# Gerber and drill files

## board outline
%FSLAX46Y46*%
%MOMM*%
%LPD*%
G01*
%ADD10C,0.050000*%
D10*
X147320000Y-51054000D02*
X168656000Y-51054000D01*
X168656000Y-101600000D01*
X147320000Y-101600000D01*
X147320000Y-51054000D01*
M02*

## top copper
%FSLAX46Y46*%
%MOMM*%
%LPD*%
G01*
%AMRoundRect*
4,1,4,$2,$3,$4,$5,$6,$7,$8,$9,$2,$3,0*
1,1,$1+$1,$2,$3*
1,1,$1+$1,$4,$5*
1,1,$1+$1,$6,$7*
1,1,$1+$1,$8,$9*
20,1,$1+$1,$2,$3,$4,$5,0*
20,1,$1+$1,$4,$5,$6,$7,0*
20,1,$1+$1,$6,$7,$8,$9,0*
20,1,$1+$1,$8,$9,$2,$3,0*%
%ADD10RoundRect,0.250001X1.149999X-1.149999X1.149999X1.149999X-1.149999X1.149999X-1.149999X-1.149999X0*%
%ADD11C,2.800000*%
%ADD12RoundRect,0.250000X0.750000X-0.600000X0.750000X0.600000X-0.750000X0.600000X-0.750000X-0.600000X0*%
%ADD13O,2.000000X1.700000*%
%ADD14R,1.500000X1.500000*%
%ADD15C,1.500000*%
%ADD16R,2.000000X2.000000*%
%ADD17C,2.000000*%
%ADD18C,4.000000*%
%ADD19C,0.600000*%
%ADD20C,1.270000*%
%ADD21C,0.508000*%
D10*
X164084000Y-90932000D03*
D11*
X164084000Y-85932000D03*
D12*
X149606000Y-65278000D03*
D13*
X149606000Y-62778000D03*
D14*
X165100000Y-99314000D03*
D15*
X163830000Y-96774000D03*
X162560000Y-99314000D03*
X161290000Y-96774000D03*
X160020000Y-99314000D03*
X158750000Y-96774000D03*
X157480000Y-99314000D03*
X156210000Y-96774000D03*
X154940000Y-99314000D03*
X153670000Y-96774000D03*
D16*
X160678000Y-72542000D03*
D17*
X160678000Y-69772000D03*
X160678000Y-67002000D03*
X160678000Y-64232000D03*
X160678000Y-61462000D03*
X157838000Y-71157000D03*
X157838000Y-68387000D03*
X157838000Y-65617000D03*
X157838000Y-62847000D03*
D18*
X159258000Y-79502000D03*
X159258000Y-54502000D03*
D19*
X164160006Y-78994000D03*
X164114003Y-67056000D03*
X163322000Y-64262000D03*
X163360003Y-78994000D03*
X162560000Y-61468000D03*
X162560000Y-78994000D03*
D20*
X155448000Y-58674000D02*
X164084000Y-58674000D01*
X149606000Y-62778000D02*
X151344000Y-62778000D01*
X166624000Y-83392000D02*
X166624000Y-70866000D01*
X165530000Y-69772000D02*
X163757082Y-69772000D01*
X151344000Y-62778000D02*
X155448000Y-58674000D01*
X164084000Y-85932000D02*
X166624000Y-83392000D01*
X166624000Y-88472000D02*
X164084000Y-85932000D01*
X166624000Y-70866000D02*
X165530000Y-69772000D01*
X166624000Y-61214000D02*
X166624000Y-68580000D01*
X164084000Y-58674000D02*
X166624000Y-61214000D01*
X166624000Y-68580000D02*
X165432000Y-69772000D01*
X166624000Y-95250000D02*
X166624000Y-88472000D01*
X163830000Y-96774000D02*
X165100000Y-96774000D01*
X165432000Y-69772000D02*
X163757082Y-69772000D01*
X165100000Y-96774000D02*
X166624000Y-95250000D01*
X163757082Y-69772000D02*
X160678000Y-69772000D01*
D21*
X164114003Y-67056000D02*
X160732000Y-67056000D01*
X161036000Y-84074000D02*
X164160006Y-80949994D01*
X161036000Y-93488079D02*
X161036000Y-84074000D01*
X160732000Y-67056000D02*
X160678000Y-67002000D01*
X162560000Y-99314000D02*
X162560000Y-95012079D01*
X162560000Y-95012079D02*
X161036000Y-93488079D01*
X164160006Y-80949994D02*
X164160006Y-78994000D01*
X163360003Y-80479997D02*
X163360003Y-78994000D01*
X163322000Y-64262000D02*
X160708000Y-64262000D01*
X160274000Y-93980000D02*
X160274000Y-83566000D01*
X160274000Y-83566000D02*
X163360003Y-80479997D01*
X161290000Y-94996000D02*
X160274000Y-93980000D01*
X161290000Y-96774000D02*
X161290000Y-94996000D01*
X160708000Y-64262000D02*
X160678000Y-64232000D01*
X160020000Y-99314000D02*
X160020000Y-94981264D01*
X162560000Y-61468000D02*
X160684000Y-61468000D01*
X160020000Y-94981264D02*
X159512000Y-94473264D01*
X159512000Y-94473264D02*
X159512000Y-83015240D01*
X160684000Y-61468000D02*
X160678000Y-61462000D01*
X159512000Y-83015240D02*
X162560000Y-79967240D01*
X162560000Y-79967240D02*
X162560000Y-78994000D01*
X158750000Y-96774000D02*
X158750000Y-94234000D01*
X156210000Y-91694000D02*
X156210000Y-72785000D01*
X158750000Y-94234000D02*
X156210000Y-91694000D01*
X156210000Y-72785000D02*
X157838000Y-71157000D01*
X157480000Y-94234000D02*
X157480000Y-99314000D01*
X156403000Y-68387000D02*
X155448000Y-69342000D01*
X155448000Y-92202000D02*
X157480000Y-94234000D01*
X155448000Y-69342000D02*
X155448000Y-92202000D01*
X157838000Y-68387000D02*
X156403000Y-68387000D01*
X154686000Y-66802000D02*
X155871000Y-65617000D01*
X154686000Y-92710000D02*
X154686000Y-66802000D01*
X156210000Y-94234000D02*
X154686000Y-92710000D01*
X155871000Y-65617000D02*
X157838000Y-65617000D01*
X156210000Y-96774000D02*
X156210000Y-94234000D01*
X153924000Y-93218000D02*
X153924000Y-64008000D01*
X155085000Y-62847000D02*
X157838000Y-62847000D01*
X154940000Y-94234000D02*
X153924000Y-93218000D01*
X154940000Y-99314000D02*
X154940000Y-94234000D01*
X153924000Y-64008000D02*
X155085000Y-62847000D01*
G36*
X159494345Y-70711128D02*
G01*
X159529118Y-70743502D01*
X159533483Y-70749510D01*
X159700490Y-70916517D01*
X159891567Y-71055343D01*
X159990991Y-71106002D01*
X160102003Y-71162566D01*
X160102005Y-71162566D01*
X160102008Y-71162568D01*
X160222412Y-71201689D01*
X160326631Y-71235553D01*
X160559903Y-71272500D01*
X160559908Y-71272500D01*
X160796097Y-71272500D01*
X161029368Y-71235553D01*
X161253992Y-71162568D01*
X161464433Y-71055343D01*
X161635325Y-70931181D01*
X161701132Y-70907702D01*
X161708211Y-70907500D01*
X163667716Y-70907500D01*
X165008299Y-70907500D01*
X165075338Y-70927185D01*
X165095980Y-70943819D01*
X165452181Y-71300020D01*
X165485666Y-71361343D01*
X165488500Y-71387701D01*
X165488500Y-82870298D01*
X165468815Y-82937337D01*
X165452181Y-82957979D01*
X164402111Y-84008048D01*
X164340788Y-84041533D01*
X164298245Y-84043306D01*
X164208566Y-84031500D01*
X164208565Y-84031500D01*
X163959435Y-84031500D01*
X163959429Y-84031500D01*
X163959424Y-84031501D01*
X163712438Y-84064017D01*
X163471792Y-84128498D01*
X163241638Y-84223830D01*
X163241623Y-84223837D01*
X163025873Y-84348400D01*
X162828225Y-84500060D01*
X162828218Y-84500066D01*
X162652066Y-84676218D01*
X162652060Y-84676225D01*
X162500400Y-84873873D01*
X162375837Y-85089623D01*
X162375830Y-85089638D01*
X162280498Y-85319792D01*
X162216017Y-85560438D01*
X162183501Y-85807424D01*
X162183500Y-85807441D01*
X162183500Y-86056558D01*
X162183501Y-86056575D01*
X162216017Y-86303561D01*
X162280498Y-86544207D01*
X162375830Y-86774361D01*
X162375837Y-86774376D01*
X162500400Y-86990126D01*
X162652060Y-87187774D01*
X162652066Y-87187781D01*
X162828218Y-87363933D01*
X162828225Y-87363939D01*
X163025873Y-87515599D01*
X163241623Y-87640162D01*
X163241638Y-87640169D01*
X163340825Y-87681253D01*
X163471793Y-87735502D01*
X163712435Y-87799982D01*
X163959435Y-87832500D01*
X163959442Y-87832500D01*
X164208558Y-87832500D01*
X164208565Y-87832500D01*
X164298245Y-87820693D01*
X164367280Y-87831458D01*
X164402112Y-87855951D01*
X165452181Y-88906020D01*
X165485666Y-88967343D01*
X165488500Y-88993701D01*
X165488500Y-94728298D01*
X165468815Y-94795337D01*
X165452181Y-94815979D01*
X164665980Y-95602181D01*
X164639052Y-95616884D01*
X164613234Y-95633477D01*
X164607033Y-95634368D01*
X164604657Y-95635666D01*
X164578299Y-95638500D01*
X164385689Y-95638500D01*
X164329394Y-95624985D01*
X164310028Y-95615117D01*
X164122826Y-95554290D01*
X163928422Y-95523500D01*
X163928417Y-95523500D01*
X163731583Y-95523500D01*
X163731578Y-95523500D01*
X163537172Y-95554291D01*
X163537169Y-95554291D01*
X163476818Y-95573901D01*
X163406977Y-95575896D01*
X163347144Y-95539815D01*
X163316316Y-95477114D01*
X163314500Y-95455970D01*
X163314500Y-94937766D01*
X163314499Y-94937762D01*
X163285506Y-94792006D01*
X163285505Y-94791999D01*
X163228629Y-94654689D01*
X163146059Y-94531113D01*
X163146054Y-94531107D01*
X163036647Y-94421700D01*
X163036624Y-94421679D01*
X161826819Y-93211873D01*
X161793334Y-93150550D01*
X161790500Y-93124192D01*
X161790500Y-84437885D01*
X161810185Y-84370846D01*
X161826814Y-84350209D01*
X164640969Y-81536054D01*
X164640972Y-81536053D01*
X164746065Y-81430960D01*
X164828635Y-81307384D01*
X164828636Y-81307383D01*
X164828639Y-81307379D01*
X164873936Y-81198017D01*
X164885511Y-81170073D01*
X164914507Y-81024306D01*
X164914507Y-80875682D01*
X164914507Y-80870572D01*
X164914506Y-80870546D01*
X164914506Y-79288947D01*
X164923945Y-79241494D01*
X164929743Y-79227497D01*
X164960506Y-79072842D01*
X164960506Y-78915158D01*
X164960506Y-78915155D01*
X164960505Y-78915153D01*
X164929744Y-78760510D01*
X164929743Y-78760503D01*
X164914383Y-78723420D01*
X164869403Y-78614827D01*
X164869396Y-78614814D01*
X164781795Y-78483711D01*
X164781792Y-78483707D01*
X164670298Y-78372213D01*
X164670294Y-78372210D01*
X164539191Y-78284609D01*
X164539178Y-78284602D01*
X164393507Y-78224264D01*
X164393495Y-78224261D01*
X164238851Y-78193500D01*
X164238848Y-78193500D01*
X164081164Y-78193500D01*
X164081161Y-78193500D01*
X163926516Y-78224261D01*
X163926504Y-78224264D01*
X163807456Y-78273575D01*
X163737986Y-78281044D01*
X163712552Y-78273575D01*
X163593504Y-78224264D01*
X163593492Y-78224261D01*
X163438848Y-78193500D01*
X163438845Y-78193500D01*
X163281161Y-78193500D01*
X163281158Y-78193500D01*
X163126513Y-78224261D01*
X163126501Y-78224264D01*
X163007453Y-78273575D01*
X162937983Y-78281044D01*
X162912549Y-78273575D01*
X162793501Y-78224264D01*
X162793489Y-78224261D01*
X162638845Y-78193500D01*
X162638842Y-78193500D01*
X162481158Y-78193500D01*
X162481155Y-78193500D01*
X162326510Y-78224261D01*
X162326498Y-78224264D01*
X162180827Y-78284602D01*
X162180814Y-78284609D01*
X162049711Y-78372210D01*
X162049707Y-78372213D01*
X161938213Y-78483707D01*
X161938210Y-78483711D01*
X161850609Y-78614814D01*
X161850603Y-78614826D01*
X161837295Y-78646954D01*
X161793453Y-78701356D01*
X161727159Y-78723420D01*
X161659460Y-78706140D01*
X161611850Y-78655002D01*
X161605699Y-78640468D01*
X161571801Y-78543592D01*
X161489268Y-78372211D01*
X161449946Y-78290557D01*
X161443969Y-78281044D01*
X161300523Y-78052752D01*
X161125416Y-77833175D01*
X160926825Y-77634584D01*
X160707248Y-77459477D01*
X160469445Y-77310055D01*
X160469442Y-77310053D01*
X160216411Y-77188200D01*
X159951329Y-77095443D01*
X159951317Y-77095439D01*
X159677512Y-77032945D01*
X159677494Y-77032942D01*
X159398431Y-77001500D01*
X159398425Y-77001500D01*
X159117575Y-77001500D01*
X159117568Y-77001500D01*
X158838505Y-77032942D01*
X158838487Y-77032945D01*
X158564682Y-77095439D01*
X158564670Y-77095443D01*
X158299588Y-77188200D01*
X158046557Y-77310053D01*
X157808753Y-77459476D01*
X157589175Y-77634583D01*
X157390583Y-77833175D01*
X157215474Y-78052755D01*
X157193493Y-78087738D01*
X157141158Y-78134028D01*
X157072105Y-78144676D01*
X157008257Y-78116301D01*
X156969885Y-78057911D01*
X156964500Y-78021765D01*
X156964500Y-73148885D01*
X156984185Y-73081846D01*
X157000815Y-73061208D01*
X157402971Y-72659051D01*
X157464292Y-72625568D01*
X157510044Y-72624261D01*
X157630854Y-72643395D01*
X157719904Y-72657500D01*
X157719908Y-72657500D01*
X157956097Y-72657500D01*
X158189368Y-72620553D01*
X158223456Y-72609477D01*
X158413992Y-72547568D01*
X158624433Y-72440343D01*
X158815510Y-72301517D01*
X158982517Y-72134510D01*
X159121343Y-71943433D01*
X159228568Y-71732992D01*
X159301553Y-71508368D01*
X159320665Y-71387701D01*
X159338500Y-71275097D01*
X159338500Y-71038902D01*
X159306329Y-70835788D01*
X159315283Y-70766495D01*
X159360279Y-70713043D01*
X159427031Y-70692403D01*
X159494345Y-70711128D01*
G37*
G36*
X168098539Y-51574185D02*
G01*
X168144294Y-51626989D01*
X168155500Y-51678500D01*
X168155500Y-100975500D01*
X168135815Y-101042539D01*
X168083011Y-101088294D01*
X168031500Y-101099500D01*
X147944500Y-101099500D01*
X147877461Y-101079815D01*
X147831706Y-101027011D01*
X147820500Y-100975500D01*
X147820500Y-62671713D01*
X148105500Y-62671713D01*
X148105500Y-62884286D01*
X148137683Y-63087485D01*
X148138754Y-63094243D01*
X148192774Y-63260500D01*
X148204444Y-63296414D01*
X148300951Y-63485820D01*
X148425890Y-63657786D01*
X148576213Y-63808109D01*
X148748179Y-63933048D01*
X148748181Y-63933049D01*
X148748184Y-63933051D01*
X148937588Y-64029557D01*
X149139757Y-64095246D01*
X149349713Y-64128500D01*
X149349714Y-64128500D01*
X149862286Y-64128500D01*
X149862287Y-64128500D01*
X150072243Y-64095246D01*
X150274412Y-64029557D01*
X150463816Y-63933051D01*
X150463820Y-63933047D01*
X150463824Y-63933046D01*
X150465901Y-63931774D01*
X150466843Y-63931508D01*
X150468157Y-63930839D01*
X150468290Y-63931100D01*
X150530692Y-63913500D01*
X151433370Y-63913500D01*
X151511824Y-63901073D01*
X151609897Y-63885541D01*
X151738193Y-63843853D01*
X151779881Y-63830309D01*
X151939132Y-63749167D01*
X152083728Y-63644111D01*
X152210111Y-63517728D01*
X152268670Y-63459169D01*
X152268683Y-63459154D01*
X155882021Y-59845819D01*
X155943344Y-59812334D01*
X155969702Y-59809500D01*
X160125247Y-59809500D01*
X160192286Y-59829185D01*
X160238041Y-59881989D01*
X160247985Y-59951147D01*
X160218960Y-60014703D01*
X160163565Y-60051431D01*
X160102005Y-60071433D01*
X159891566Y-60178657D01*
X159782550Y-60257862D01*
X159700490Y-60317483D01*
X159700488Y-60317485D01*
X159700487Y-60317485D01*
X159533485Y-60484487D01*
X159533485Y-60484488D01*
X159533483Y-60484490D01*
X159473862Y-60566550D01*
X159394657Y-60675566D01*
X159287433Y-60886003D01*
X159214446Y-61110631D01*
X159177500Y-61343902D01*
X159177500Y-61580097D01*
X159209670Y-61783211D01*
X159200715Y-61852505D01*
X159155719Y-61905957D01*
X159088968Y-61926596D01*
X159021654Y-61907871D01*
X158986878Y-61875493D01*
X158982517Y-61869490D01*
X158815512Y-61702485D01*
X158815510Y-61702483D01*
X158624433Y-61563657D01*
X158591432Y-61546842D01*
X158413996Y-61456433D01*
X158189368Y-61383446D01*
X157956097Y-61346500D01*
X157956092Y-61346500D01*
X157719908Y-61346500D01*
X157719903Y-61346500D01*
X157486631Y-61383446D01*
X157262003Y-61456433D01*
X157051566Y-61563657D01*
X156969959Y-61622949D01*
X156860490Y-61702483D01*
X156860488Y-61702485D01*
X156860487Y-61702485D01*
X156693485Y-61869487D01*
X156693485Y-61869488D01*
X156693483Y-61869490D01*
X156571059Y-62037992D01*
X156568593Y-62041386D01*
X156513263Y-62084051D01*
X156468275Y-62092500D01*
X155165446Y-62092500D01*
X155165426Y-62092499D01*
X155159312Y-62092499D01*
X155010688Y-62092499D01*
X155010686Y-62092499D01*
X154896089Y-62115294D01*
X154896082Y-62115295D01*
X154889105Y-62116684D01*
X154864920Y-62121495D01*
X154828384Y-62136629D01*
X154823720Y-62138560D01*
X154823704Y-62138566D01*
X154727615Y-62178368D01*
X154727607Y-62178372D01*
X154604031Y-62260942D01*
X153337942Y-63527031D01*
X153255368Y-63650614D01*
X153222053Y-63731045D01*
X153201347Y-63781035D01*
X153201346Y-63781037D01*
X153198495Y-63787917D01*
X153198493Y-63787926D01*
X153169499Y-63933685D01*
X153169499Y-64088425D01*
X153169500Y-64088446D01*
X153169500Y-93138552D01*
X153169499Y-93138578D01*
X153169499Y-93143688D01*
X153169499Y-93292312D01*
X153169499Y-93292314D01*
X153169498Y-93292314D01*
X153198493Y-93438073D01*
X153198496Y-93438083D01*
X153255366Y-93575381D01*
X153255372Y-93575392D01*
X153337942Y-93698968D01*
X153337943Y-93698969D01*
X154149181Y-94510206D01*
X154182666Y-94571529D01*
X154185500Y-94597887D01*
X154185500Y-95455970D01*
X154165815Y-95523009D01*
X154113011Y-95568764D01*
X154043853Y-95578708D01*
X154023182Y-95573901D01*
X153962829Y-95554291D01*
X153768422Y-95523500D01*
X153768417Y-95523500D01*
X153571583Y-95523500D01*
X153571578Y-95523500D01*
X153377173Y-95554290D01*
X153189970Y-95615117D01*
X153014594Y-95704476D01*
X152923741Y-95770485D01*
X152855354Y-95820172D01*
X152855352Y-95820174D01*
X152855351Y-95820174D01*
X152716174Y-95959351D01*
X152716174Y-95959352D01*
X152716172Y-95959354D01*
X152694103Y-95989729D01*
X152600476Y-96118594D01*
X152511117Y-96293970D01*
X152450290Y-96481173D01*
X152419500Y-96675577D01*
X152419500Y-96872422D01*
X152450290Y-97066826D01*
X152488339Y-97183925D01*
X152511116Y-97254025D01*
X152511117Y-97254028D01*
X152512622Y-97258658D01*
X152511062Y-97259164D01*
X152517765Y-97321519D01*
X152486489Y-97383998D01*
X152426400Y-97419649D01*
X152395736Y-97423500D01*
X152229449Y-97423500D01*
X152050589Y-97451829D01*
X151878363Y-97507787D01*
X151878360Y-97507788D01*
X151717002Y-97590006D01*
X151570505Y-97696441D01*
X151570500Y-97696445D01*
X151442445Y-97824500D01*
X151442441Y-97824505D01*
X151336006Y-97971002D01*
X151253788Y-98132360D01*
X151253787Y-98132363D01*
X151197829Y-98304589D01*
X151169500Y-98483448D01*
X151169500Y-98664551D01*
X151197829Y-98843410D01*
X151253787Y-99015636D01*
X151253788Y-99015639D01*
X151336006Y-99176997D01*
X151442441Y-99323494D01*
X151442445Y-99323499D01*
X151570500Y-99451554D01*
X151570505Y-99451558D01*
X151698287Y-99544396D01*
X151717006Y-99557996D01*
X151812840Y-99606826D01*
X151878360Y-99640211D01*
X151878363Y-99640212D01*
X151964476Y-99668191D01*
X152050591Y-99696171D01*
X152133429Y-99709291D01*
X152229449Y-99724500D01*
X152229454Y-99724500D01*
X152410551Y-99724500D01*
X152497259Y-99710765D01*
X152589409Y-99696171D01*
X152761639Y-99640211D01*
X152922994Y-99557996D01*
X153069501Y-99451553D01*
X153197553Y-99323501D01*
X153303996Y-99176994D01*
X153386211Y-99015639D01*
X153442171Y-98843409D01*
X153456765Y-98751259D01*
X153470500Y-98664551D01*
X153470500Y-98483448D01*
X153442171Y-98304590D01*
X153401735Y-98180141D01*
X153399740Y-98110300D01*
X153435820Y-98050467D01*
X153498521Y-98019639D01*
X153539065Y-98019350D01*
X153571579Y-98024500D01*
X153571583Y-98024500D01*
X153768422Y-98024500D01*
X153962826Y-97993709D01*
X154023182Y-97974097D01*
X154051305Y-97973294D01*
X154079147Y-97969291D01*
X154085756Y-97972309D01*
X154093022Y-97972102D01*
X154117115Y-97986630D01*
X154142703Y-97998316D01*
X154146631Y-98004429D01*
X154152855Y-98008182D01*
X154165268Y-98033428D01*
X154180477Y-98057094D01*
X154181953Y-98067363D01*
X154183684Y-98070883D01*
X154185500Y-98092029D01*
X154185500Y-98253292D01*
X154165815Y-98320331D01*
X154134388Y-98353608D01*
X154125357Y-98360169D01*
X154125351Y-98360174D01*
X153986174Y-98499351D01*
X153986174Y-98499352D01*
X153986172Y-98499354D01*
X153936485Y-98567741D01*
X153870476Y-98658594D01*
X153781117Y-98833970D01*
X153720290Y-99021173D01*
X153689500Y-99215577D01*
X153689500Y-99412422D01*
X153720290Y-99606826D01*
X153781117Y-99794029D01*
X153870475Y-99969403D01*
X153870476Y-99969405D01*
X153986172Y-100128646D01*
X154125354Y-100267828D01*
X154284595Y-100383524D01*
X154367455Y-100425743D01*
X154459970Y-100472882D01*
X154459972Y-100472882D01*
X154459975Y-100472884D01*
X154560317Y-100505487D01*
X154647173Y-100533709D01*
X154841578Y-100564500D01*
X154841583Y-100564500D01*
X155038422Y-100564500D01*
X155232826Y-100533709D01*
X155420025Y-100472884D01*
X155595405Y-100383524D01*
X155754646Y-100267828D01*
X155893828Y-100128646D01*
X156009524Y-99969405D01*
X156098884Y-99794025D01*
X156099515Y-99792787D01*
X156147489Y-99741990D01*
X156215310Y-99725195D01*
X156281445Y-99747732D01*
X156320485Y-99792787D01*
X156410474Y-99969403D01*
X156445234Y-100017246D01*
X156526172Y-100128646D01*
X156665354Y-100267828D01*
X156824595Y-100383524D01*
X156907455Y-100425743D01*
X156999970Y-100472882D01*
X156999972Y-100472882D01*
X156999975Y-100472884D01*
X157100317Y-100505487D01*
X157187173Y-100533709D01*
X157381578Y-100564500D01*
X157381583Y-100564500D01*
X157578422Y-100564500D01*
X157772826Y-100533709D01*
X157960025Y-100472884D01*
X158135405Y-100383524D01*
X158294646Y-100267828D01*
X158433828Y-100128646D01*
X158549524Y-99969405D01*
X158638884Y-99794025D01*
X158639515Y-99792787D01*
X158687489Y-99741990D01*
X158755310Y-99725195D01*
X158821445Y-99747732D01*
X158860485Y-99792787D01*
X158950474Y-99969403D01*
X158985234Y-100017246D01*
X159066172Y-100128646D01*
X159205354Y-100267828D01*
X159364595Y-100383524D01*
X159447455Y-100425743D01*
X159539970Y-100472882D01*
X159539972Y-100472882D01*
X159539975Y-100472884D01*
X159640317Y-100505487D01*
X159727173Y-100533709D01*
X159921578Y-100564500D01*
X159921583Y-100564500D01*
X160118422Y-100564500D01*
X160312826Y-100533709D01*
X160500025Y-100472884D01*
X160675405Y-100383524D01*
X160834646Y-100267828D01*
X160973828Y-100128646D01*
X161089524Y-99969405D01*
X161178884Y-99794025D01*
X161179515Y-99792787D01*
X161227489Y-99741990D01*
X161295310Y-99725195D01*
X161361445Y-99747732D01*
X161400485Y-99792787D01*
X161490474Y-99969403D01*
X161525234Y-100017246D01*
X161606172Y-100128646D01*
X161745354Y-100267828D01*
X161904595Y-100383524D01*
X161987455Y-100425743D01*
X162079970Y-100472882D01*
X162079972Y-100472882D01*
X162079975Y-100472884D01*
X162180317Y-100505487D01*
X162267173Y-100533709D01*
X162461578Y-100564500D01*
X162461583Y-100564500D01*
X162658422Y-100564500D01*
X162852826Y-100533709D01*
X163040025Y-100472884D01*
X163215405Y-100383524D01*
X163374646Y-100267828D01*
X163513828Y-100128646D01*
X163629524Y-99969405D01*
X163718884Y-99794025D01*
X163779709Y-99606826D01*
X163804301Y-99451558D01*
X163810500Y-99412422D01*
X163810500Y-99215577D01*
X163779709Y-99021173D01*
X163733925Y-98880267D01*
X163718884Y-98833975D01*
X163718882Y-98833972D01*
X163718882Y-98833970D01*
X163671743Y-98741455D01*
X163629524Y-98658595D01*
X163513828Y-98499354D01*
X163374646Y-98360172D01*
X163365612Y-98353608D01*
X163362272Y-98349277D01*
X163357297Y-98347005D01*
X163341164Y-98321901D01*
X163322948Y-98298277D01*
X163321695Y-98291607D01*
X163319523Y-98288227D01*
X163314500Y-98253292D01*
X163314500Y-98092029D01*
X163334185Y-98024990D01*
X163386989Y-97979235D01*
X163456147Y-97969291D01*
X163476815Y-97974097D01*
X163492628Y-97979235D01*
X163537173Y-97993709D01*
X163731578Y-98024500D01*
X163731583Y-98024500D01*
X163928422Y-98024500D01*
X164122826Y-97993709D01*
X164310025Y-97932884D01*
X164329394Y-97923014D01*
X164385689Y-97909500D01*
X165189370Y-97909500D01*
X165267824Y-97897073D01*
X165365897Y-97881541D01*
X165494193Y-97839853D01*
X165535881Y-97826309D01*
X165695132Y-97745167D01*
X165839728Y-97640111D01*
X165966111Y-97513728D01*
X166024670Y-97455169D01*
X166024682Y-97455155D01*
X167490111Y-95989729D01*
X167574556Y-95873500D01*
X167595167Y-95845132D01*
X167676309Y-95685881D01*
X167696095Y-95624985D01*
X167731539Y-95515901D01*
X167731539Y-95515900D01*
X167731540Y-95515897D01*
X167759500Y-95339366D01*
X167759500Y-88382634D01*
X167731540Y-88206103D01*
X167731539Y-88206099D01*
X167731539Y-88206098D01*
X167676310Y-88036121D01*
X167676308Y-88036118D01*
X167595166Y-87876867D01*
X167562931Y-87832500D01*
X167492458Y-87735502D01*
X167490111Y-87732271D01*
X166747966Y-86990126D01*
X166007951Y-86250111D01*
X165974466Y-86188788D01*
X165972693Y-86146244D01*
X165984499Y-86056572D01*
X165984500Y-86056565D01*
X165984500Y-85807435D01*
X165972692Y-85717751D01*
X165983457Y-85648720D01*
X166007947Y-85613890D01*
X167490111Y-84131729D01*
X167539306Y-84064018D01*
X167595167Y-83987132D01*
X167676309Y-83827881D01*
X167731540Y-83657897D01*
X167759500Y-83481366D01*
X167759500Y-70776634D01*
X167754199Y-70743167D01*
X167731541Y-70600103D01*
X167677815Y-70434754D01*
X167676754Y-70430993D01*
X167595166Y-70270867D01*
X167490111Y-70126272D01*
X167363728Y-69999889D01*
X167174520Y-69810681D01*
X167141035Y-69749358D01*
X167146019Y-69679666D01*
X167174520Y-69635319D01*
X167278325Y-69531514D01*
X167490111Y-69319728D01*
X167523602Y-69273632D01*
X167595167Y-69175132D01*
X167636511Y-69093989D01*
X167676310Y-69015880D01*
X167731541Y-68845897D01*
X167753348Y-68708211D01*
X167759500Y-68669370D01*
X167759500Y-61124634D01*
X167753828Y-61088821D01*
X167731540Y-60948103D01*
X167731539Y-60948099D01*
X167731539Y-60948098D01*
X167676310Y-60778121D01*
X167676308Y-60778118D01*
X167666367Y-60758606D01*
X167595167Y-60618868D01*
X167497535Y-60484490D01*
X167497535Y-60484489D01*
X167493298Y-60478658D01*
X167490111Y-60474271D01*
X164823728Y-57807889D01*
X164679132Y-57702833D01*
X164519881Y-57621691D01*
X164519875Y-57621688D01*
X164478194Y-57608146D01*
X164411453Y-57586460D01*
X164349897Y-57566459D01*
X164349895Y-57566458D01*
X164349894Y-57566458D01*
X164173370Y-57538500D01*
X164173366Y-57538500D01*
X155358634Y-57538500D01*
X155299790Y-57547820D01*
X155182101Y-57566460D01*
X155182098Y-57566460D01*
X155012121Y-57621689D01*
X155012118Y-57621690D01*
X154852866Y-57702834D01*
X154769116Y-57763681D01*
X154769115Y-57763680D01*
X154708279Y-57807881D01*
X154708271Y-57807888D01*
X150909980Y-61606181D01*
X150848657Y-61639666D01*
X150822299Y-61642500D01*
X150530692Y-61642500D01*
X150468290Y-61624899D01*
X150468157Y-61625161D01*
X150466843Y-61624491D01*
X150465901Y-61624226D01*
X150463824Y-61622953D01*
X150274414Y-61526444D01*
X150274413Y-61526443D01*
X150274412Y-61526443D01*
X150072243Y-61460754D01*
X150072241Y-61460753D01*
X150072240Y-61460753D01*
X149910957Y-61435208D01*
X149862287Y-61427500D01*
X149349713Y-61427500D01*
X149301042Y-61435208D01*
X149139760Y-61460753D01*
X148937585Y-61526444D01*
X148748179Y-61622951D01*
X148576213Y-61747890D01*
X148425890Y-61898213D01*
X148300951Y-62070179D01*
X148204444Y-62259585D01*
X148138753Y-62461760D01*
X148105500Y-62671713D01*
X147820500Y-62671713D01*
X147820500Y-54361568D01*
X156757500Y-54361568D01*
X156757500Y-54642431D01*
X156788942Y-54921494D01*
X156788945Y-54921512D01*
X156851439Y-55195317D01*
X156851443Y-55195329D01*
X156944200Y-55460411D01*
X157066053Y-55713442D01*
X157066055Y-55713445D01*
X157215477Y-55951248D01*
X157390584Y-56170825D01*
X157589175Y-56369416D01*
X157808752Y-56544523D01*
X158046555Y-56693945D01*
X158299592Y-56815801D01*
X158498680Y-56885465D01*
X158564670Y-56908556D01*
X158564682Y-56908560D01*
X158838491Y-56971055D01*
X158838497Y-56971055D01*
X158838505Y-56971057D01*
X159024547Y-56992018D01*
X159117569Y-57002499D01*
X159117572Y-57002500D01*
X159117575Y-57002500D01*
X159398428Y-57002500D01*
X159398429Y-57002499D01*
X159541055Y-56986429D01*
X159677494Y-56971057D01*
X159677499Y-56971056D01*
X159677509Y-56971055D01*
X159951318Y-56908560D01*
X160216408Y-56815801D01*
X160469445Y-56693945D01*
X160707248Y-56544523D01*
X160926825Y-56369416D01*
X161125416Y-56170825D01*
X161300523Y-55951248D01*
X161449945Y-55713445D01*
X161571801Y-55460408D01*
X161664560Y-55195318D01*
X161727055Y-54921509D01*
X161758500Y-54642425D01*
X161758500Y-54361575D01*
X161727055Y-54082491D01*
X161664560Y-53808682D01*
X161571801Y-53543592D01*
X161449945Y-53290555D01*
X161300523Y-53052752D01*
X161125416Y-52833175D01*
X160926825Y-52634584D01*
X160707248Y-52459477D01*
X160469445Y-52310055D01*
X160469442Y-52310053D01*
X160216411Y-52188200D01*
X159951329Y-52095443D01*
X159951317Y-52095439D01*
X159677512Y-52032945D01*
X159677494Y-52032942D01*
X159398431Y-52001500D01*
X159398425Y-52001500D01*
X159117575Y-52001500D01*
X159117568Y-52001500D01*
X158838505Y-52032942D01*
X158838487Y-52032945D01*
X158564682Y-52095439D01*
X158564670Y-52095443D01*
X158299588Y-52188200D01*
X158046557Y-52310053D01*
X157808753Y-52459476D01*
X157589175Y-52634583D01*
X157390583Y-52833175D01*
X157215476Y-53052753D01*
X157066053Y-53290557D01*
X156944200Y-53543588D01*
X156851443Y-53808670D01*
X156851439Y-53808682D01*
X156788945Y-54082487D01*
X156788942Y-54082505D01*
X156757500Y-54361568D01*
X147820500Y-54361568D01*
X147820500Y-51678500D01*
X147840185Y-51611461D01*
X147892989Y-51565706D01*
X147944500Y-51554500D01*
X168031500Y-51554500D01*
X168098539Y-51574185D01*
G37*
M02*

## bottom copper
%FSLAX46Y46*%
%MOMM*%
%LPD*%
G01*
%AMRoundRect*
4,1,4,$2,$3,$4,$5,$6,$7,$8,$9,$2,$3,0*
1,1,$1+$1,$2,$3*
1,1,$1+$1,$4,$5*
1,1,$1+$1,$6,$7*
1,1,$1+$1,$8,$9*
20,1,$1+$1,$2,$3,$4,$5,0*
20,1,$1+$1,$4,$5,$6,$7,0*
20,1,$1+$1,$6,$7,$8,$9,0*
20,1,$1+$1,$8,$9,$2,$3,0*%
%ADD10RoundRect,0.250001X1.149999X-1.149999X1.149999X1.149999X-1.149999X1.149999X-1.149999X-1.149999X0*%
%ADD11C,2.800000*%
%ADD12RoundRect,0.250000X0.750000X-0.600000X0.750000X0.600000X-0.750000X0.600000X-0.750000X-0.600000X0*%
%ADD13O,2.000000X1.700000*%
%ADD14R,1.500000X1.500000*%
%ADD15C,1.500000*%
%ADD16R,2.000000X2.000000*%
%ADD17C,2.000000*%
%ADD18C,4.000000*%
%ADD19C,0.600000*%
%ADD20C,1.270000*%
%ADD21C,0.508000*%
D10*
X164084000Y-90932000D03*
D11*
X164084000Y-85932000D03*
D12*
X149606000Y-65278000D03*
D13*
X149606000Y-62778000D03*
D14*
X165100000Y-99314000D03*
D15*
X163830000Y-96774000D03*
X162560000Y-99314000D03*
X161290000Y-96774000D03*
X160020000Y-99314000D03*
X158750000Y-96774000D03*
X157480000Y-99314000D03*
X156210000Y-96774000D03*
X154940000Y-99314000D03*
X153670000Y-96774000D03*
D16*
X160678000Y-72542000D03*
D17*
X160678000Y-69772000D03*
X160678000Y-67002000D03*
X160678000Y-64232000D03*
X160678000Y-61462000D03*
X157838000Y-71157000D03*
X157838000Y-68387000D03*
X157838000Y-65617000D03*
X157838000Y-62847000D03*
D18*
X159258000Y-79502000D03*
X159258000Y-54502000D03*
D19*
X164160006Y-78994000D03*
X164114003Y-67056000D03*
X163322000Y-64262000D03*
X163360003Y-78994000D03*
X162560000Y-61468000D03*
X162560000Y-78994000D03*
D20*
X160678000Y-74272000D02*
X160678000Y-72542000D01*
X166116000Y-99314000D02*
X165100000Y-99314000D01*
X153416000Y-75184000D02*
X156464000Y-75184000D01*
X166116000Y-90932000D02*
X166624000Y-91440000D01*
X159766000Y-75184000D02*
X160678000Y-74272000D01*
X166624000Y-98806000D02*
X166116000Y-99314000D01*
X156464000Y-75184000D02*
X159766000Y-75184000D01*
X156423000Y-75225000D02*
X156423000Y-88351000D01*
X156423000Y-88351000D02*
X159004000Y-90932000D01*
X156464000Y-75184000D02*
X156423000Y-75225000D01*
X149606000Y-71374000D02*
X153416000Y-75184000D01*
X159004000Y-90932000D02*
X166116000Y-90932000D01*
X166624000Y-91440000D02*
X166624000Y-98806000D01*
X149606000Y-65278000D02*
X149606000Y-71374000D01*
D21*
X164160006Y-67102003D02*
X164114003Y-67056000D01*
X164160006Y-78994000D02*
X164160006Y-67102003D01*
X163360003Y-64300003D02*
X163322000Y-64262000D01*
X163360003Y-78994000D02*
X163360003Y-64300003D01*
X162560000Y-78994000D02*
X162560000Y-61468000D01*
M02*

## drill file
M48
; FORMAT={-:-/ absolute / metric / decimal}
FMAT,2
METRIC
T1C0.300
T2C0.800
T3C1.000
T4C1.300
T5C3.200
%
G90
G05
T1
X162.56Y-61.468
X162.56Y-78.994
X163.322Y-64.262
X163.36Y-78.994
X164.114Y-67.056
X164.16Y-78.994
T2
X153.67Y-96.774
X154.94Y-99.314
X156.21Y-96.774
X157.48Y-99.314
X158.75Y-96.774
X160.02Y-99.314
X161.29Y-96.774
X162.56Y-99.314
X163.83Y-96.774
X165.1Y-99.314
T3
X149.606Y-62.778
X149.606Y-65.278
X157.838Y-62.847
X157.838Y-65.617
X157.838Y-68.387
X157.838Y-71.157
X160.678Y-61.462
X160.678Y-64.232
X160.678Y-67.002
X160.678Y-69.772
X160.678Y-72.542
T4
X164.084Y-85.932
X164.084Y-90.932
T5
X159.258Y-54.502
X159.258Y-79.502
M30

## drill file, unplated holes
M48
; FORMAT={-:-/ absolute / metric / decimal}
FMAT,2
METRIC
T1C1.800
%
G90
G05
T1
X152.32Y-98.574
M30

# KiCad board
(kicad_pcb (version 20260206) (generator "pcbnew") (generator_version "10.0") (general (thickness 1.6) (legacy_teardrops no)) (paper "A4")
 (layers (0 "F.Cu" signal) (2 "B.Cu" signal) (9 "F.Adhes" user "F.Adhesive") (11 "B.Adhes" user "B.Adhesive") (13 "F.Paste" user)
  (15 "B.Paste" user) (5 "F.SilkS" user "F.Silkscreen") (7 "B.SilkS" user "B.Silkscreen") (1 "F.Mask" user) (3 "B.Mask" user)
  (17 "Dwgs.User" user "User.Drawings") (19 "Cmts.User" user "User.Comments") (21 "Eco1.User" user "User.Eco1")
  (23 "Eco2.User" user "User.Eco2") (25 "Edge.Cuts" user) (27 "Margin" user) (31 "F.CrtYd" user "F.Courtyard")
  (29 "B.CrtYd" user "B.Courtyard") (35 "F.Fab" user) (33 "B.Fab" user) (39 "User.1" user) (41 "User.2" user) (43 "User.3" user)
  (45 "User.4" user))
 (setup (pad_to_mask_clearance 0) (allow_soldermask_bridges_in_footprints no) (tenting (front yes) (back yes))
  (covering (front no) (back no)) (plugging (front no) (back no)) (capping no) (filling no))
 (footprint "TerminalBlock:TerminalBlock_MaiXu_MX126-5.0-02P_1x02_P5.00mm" (layer "F.Cu") (at 164.084 90.932 90)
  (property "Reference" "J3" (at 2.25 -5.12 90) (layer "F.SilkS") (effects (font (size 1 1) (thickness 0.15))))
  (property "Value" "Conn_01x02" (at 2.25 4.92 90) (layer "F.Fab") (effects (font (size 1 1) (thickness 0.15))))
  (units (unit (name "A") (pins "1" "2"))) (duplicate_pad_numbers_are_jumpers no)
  (pad "1" thru_hole roundrect (at 0 0 90) (size 2.8 2.8) (drill 1.3) (layers "*.Cu" "*.Mask") (remove_unused_layers no)
   (roundrect_rratio 0.089286) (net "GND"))
  (pad "2" thru_hole circle (at 5 0 90) (size 2.8 2.8) (drill 1.3) (layers "*.Cu" "*.Mask") (remove_unused_layers no) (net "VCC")))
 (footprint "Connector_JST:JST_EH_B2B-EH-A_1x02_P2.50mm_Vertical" (layer "F.Cu") (at 149.606 65.278 90)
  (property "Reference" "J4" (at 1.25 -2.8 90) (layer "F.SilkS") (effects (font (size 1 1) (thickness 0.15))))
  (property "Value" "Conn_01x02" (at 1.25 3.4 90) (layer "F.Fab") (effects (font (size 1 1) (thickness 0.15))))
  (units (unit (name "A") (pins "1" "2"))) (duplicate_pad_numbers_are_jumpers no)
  (pad "1" thru_hole roundrect (at 0 0 90) (size 1.7 2) (drill 1) (layers "*.Cu" "*.Mask") (remove_unused_layers no)
   (roundrect_rratio 0.147059) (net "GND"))
  (pad "2" thru_hole oval (at 2.5 0 90) (size 1.7 2) (drill 1) (layers "*.Cu" "*.Mask") (remove_unused_layers no) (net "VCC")))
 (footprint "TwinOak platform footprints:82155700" (layer "F.Cu") (at 165.1 99.314 180)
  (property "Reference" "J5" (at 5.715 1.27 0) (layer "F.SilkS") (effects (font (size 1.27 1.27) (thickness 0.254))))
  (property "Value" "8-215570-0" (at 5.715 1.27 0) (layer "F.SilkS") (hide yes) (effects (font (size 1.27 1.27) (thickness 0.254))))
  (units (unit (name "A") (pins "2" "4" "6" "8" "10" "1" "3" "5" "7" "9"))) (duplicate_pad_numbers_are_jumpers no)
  (pad "" np_thru_hole circle (at 12.78 0.74 180) (size 1.8 1.8) (drill 1.8) (layers "*.Cu" "*.Mask"))
  (pad "1" thru_hole rect (at 0 0 180) (size 1.5 1.5) (drill 0.8) (layers "*.Cu" "*.Mask") (remove_unused_layers no) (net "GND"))
  (pad "2" thru_hole circle (at 1.27 2.54 180) (size 1.5 1.5) (drill 0.8) (layers "*.Cu" "*.Mask") (remove_unused_layers no) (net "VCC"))
  (pad "3" thru_hole circle (at 2.54 0 180) (size 1.5 1.5) (drill 0.8) (layers "*.Cu" "*.Mask") (remove_unused_layers no)
   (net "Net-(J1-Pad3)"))
  (pad "4" thru_hole circle (at 3.81 2.54 180) (size 1.5 1.5) (drill 0.8) (layers "*.Cu" "*.Mask") (remove_unused_layers no)
   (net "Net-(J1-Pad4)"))
  (pad "5" thru_hole circle (at 5.08 0 180) (size 1.5 1.5) (drill 0.8) (layers "*.Cu" "*.Mask") (remove_unused_layers no)
   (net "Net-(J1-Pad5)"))
  (pad "6" thru_hole circle (at 6.35 2.54 180) (size 1.5 1.5) (drill 0.8) (layers "*.Cu" "*.Mask") (remove_unused_layers no)
   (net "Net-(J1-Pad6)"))
  (pad "7" thru_hole circle (at 7.62 0 180) (size 1.5 1.5) (drill 0.8) (layers "*.Cu" "*.Mask") (remove_unused_layers no)
   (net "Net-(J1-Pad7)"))
  (pad "8" thru_hole circle (at 8.89 2.54 180) (size 1.5 1.5) (drill 0.8) (layers "*.Cu" "*.Mask") (remove_unused_layers no)
   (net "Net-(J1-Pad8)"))
  (pad "9" thru_hole circle (at 10.16 0 180) (size 1.5 1.5) (drill 0.8) (layers "*.Cu" "*.Mask") (remove_unused_layers no)
   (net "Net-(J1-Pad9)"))
  (pad "10" thru_hole circle (at 11.43 2.54 180) (size 1.5 1.5) (drill 0.8) (layers "*.Cu" "*.Mask") (remove_unused_layers no)
   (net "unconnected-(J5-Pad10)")))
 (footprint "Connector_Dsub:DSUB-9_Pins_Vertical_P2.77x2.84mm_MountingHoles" (layer "B.Cu") (at 160.678 72.542 90)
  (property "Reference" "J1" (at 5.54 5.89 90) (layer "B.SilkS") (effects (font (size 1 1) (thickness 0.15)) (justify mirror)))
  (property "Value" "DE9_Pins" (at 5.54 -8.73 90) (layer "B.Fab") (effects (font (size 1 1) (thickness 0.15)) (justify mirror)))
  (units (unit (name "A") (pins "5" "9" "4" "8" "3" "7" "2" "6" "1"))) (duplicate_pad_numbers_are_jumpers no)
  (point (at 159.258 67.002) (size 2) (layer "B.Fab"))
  (pad "1" thru_hole rect (at 0 0 90) (size 2 2) (drill 1) (layers "*.Cu" "*.Mask") (remove_unused_layers no) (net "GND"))
  (pad "2" thru_hole circle (at 2.77 0 90) (size 2 2) (drill 1) (layers "*.Cu" "*.Mask") (remove_unused_layers no) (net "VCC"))
  (pad "3" thru_hole circle (at 5.54 0 90) (size 2 2) (drill 1) (layers "*.Cu" "*.Mask") (remove_unused_layers no) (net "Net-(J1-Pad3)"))
  (pad "4" thru_hole circle (at 8.31 0 90) (size 2 2) (drill 1) (layers "*.Cu" "*.Mask") (remove_unused_layers no) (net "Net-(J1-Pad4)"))
  (pad "5" thru_hole circle (at 11.08 0 90) (size 2 2) (drill 1) (layers "*.Cu" "*.Mask") (remove_unused_layers no) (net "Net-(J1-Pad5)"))
  (pad "6" thru_hole circle (at 1.385 -2.84 90) (size 2 2) (drill 1) (layers "*.Cu" "*.Mask") (remove_unused_layers no)
   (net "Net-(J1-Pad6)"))
  (pad "7" thru_hole circle (at 4.155 -2.84 90) (size 2 2) (drill 1) (layers "*.Cu" "*.Mask") (remove_unused_layers no)
   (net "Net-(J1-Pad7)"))
  (pad "8" thru_hole circle (at 6.925 -2.84 90) (size 2 2) (drill 1) (layers "*.Cu" "*.Mask") (remove_unused_layers no)
   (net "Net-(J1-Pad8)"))
  (pad "9" thru_hole circle (at 9.695 -2.84 90) (size 2 2) (drill 1) (layers "*.Cu" "*.Mask") (remove_unused_layers no)
   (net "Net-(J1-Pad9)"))
  (pad "SH" thru_hole circle (at -6.96 -1.42 90) (size 4 4) (drill 3.2) (layers "*.Cu" "*.Mask") (remove_unused_layers no))
  (pad "SH" thru_hole circle (at 18.04 -1.42 90) (size 4 4) (drill 3.2) (layers "*.Cu" "*.Mask") (remove_unused_layers no)))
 (gr_rect (start 147.32 51.054) (end 168.656 101.6) (stroke (width 0.05) (type default)) (fill no) (layer "Edge.Cuts"))
 (segment (start 160.678 74.272) (end 160.678 72.542) (width 1.27) (layer "B.Cu") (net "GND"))
 (segment (start 166.116 99.314) (end 165.1 99.314) (width 1.27) (layer "B.Cu") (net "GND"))
 (segment (start 153.416 75.184) (end 156.464 75.184) (width 1.27) (layer "B.Cu") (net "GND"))
 (segment (start 166.116 90.932) (end 166.624 91.44) (width 1.27) (layer "B.Cu") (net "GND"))
 (segment (start 159.766 75.184) (end 160.678 74.272) (width 1.27) (layer "B.Cu") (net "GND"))
 (segment (start 166.624 98.806) (end 166.116 99.314) (width 1.27) (layer "B.Cu") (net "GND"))
 (segment (start 156.464 75.184) (end 159.766 75.184) (width 1.27) (layer "B.Cu") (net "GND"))
 (segment (start 156.423 75.225) (end 156.423 88.351) (width 1.27) (layer "B.Cu") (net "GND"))
 (segment (start 156.423 88.351) (end 159.004 90.932) (width 1.27) (layer "B.Cu") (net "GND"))
 (segment (start 156.464 75.184) (end 156.423 75.225) (width 1.27) (layer "B.Cu") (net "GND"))
 (segment (start 149.606 71.374) (end 153.416 75.184) (width 1.27) (layer "B.Cu") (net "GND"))
 (segment (start 159.004 90.932) (end 166.116 90.932) (width 1.27) (layer "B.Cu") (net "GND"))
 (segment (start 166.624 91.44) (end 166.624 98.806) (width 1.27) (layer "B.Cu") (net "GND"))
 (segment (start 149.606 65.278) (end 149.606 71.374) (width 1.27) (layer "B.Cu") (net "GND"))
 (segment (start 155.448 58.674) (end 164.084 58.674) (width 1.27) (layer "F.Cu") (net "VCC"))
 (segment (start 149.606 62.778) (end 151.344 62.778) (width 1.27) (layer "F.Cu") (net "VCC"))
 (segment (start 166.624 83.392) (end 166.624 70.866) (width 1.27) (layer "F.Cu") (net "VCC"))
 (segment (start 165.53 69.772) (end 163.757082 69.772) (width 1.27) (layer "F.Cu") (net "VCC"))
 (segment (start 151.344 62.778) (end 155.448 58.674) (width 1.27) (layer "F.Cu") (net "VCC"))
 (segment (start 164.084 85.932) (end 166.624 83.392) (width 1.27) (layer "F.Cu") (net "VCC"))
 (segment (start 166.624 88.472) (end 164.084 85.932) (width 1.27) (layer "F.Cu") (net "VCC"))
 (segment (start 166.624 70.866) (end 165.53 69.772) (width 1.27) (layer "F.Cu") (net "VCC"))
 (segment (start 166.624 61.214) (end 166.624 68.58) (width 1.27) (layer "F.Cu") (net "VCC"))
 (segment (start 164.084 58.674) (end 166.624 61.214) (width 1.27) (layer "F.Cu") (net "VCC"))
 (segment (start 166.624 68.58) (end 165.432 69.772) (width 1.27) (layer "F.Cu") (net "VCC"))
 (segment (start 166.624 95.25) (end 166.624 88.472) (width 1.27) (layer "F.Cu") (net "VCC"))
 (segment (start 163.83 96.774) (end 165.1 96.774) (width 1.27) (layer "F.Cu") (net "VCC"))
 (segment (start 165.432 69.772) (end 163.757082 69.772) (width 1.27) (layer "F.Cu") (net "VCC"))
 (segment (start 165.1 96.774) (end 166.624 95.25) (width 1.27) (layer "F.Cu") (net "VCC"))
 (segment (start 163.757082 69.772) (end 160.678 69.772) (width 1.27) (layer "F.Cu") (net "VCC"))
 (segment (start 164.114003 67.056) (end 160.732 67.056) (width 0.508) (layer "F.Cu") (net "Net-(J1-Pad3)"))
 (segment (start 161.036 84.074) (end 164.160006 80.949994) (width 0.508) (layer "F.Cu") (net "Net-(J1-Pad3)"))
 (segment (start 161.036 93.488079) (end 161.036 84.074) (width 0.508) (layer "F.Cu") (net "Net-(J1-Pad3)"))
 (segment (start 160.732 67.056) (end 160.678 67.002) (width 0.508) (layer "F.Cu") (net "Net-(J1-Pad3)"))
 (segment (start 162.56 99.314) (end 162.56 95.012079) (width 0.508) (layer "F.Cu") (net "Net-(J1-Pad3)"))
 (segment (start 162.56 95.012079) (end 161.036 93.488079) (width 0.508) (layer "F.Cu") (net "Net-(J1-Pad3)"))
 (segment (start 164.160006 80.949994) (end 164.160006 78.994) (width 0.508) (layer "F.Cu") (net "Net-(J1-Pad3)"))
 (via (at 164.160006 78.994) (size 0.6) (drill 0.3) (layers "F.Cu" "B.Cu") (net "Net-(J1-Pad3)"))
 (via (at 164.114003 67.056) (size 0.6) (drill 0.3) (layers "F.Cu" "B.Cu") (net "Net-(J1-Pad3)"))
 (segment (start 164.160006 67.102003) (end 164.114003 67.056) (width 0.508) (layer "B.Cu") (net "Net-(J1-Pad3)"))
 (segment (start 164.160006 78.994) (end 164.160006 67.102003) (width 0.508) (layer "B.Cu") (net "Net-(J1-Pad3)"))
 (segment (start 163.360003 80.479997) (end 163.360003 78.994) (width 0.508) (layer "F.Cu") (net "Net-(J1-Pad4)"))
 (segment (start 163.322 64.262) (end 160.708 64.262) (width 0.508) (layer "F.Cu") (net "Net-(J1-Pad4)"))
 (segment (start 160.274 93.98) (end 160.274 83.566) (width 0.508) (layer "F.Cu") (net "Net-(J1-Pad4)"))
 (segment (start 160.274 83.566) (end 163.360003 80.479997) (width 0.508) (layer "F.Cu") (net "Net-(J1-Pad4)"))
 (segment (start 161.29 94.996) (end 160.274 93.98) (width 0.508) (layer "F.Cu") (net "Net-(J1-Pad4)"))
 (segment (start 161.29 96.774) (end 161.29 94.996) (width 0.508) (layer "F.Cu") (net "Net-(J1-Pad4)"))
 (segment (start 160.708 64.262) (end 160.678 64.232) (width 0.508) (layer "F.Cu") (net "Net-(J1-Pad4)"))
 (via (at 163.322 64.262) (size 0.6) (drill 0.3) (layers "F.Cu" "B.Cu") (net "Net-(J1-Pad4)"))
 (via (at 163.360003 78.994) (size 0.6) (drill 0.3) (layers "F.Cu" "B.Cu") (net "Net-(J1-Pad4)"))
 (segment (start 163.360003 64.300003) (end 163.322 64.262) (width 0.508) (layer "B.Cu") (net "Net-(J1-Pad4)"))
 (segment (start 163.360003 78.994) (end 163.360003 64.300003) (width 0.508) (layer "B.Cu") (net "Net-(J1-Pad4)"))
 (segment (start 160.02 99.314) (end 160.02 94.981264) (width 0.508) (layer "F.Cu") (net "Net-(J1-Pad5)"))
 (segment (start 162.56 61.468) (end 160.684 61.468) (width 0.508) (layer "F.Cu") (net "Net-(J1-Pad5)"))
 (segment (start 160.02 94.981264) (end 159.512 94.473264) (width 0.508) (layer "F.Cu") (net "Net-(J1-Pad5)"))
 (segment (start 159.512 94.473264) (end 159.512 83.01524) (width 0.508) (layer "F.Cu") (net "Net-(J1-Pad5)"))
 (segment (start 160.684 61.468) (end 160.678 61.462) (width 0.508) (layer "F.Cu") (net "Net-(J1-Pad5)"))
 (segment (start 159.512 83.01524) (end 162.56 79.96724) (width 0.508) (layer "F.Cu") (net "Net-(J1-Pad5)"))
 (segment (start 162.56 79.96724) (end 162.56 78.994) (width 0.508) (layer "F.Cu") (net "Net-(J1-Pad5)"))
 (via (at 162.56 61.468) (size 0.6) (drill 0.3) (layers "F.Cu" "B.Cu") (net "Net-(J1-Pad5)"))
 (via (at 162.56 78.994) (size 0.6) (drill 0.3) (layers "F.Cu" "B.Cu") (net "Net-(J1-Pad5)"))
 (segment (start 162.56 78.994) (end 162.56 61.468) (width 0.508) (layer "B.Cu") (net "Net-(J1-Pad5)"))
 (segment (start 158.75 96.774) (end 158.75 94.234) (width 0.508) (layer "F.Cu") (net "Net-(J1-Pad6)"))
 (segment (start 156.21 91.694) (end 156.21 72.785) (width 0.508) (layer "F.Cu") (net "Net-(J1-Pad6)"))
 (segment (start 158.75 94.234) (end 156.21 91.694) (width 0.508) (layer "F.Cu") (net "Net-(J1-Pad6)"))
 (segment (start 156.21 72.785) (end 157.838 71.157) (width 0.508) (layer "F.Cu") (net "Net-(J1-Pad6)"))
 (segment (start 157.48 94.234) (end 157.48 99.314) (width 0.508) (layer "F.Cu") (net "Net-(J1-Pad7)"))
 (segment (start 156.403 68.387) (end 155.448 69.342) (width 0.508) (layer "F.Cu") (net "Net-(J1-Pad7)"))
 (segment (start 155.448 92.202) (end 157.48 94.234) (width 0.508) (layer "F.Cu") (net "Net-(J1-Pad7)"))
 (segment (start 155.448 69.342) (end 155.448 92.202) (width 0.508) (layer "F.Cu") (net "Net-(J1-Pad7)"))
 (segment (start 157.838 68.387) (end 156.403 68.387) (width 0.508) (layer "F.Cu") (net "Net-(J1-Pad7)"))
 (segment (start 154.686 66.802) (end 155.871 65.617) (width 0.508) (layer "F.Cu") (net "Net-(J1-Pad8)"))
 (segment (start 154.686 92.71) (end 154.686 66.802) (width 0.508) (layer "F.Cu") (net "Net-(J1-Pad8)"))
 (segment (start 156.21 94.234) (end 154.686 92.71) (width 0.508) (layer "F.Cu") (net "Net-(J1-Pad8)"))
 (segment (start 155.871 65.617) (end 157.838 65.617) (width 0.508) (layer "F.Cu") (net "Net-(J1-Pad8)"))
 (segment (start 156.21 96.774) (end 156.21 94.234) (width 0.508) (layer "F.Cu") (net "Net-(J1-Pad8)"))
 (segment (start 153.924 93.218) (end 153.924 64.008) (width 0.508) (layer "F.Cu") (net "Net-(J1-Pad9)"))
 (segment (start 155.085 62.847) (end 157.838 62.847) (width 0.508) (layer "F.Cu") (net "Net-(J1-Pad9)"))
 (segment (start 154.94 94.234) (end 153.924 93.218) (width 0.508) (layer "F.Cu") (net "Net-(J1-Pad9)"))
 (segment (start 154.94 99.314) (end 154.94 94.234) (width 0.508) (layer "F.Cu") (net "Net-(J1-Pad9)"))
 (segment (start 153.924 64.008) (end 155.085 62.847) (width 0.508) (layer "F.Cu") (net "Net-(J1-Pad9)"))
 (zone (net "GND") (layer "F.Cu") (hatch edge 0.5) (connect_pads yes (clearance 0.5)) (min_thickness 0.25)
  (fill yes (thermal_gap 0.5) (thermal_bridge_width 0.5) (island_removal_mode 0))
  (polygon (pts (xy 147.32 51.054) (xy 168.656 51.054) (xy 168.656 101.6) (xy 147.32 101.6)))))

